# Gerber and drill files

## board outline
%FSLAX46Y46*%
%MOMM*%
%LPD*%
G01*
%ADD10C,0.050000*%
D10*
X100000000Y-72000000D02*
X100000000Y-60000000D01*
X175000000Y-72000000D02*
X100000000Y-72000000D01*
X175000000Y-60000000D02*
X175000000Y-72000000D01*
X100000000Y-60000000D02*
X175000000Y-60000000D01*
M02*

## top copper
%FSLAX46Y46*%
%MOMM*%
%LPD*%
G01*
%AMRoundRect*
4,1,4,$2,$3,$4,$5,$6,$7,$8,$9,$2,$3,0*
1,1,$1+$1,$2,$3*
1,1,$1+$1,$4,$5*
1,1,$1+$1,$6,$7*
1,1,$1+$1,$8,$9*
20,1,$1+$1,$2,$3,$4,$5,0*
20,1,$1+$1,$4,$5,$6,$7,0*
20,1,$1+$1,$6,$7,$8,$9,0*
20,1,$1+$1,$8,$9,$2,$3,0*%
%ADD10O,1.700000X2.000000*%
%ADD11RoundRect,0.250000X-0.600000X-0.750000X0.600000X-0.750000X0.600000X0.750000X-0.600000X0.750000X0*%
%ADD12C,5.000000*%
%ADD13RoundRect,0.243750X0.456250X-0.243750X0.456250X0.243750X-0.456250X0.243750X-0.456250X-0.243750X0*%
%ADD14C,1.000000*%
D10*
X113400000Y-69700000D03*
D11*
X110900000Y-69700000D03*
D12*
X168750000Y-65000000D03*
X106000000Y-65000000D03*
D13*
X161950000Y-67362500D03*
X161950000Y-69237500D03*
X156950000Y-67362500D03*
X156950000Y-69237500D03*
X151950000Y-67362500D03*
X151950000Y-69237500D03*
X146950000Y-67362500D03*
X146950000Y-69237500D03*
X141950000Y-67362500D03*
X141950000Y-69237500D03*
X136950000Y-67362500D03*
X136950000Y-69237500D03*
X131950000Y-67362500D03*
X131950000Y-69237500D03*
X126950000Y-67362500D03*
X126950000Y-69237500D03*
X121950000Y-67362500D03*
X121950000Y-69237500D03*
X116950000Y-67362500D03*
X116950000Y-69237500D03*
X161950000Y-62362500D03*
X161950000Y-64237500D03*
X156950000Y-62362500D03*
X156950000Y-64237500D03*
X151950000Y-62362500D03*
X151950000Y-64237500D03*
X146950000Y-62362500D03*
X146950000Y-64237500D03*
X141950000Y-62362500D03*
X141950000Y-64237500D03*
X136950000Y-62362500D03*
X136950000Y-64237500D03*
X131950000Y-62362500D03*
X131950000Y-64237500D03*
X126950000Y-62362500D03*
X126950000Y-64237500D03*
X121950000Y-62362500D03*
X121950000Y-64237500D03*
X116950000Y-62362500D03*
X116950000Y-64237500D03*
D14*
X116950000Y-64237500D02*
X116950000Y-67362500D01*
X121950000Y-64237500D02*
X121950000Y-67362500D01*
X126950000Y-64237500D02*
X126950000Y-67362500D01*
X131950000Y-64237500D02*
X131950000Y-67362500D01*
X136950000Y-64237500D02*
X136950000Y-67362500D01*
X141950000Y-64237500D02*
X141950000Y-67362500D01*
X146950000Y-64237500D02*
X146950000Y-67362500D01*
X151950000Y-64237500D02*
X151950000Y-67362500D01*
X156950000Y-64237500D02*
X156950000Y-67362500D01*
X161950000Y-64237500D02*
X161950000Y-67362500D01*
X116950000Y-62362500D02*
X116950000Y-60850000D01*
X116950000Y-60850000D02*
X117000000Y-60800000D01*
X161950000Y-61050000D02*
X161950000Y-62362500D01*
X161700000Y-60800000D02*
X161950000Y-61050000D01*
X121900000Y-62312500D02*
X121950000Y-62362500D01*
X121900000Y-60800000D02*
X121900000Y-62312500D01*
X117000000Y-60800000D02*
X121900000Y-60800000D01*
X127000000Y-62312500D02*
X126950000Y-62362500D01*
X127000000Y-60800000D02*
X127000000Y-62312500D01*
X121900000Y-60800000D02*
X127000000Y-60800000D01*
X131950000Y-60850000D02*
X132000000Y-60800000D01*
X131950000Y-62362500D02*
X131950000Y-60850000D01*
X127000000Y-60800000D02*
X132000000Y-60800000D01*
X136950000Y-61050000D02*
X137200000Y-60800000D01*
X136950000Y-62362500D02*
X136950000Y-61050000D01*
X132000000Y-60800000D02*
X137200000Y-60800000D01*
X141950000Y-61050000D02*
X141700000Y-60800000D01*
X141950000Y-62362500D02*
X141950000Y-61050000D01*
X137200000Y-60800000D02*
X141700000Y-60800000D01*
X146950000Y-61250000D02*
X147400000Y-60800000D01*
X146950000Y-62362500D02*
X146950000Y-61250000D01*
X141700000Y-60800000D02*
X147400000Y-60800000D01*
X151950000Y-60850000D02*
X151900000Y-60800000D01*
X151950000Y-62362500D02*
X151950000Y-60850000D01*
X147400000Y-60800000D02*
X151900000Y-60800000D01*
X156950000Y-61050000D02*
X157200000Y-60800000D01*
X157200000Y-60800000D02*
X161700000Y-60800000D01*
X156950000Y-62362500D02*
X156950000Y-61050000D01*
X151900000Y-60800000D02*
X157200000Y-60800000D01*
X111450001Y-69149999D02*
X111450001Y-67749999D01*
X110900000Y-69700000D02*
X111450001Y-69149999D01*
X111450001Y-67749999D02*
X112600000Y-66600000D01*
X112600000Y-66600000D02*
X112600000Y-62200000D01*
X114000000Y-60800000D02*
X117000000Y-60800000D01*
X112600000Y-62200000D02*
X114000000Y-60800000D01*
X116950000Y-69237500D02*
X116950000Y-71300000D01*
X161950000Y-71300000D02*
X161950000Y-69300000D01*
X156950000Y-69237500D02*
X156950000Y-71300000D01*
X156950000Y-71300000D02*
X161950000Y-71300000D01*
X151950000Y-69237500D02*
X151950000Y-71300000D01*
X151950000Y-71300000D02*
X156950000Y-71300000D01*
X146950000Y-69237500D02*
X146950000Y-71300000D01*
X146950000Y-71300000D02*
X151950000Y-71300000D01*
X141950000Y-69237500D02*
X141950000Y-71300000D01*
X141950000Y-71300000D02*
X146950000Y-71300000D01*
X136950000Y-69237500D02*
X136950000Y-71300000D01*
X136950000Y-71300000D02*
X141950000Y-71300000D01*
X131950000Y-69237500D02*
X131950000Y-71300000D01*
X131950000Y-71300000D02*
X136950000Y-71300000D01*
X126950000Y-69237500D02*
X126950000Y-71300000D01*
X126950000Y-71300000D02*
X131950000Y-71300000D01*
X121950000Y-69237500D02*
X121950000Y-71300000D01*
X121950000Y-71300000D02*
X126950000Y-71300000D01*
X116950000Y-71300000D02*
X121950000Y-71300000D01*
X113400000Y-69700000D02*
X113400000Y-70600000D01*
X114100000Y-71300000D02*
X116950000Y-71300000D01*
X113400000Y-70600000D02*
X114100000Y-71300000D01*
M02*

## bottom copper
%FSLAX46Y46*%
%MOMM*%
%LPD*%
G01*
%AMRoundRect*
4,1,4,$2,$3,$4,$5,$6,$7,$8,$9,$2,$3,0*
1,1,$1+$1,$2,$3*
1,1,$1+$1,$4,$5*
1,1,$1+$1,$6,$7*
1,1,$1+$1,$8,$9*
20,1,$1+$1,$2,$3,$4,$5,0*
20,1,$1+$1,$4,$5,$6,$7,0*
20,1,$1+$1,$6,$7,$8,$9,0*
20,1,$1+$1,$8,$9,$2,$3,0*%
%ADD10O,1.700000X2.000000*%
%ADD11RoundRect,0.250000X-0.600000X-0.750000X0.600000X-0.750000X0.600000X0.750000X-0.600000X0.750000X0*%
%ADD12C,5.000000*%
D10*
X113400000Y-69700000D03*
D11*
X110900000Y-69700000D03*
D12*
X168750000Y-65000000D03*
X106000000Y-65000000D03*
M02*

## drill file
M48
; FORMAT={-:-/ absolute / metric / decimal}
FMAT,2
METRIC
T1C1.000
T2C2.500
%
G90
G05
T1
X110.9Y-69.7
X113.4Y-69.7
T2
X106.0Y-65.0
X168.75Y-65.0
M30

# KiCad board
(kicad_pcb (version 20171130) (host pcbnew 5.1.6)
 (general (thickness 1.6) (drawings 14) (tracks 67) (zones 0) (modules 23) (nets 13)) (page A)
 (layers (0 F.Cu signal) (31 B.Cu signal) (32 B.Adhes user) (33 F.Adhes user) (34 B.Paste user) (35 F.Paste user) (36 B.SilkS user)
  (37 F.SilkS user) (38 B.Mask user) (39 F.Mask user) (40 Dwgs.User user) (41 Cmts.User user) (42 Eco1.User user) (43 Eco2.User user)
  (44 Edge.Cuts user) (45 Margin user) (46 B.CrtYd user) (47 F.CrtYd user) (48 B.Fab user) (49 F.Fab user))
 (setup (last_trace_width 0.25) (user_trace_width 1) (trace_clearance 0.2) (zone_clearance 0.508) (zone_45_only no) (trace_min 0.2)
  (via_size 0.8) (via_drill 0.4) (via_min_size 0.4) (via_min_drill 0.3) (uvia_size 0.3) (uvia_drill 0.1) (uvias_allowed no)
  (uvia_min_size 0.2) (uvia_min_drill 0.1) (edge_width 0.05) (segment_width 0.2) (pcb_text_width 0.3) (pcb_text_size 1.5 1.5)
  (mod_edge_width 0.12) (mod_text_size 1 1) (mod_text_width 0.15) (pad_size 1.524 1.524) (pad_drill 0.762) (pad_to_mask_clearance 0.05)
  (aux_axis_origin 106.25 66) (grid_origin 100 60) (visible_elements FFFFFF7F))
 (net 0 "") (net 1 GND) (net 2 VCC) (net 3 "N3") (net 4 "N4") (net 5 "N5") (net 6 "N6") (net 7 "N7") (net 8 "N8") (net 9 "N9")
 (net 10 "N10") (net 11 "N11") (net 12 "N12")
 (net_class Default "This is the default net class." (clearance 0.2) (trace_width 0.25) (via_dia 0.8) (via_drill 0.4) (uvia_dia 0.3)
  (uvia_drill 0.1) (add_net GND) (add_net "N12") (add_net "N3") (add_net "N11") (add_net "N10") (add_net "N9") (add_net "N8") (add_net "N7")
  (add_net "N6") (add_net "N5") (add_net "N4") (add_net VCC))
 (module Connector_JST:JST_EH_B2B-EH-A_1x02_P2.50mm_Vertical (layer F.Cu) (at 110.9 69.7)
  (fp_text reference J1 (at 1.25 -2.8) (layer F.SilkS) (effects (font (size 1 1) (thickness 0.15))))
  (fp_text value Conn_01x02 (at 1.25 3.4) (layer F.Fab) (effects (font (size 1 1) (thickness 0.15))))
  (pad 2 thru_hole oval (at 2.5 0) (size 1.7 2) (drill 1) (layers *.Cu *.Mask) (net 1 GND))
  (pad 1 thru_hole roundrect (at 0 0) (size 1.7 2) (drill 1) (layers *.Cu *.Mask) (roundrect_rratio 0.147059) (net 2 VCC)))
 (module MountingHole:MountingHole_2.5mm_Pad (layer F.Cu) (at 168.75 65)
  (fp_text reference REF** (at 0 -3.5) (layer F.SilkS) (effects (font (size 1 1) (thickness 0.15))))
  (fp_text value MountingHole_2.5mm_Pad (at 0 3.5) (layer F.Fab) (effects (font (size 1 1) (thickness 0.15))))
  (pad 1 thru_hole circle (at 0 0) (size 5 5) (drill 2.5) (layers *.Cu *.Mask)))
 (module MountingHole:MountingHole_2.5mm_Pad (layer F.Cu) (at 106 65)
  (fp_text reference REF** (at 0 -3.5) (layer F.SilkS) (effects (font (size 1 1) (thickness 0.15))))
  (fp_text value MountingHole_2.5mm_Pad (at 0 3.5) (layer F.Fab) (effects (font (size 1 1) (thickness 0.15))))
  (pad 1 thru_hole circle (at 0 0) (size 5 5) (drill 2.5) (layers *.Cu *.Mask)))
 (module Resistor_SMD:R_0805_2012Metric (layer F.Cu) (at 161.95 68.3 90)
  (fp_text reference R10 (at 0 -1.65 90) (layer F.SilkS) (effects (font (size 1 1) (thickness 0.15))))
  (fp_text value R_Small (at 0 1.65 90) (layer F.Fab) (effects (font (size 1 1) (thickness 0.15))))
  (pad 2 smd roundrect (at 0.9375 0 90) (size 0.975 1.4) (layers F.Cu F.Paste F.Mask) (roundrect_rratio 0.25) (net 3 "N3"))
  (pad 1 smd roundrect (at -0.9375 0 90) (size 0.975 1.4) (layers F.Cu F.Paste F.Mask) (roundrect_rratio 0.25) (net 1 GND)))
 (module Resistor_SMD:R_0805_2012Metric (layer F.Cu) (at 156.95 68.3 90)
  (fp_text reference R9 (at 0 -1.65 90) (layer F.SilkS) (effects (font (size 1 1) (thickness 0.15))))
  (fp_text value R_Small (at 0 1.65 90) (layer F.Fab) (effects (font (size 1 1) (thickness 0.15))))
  (pad 2 smd roundrect (at 0.9375 0 90) (size 0.975 1.4) (layers F.Cu F.Paste F.Mask) (roundrect_rratio 0.25) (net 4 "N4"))
  (pad 1 smd roundrect (at -0.9375 0 90) (size 0.975 1.4) (layers F.Cu F.Paste F.Mask) (roundrect_rratio 0.25) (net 1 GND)))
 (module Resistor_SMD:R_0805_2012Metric (layer F.Cu) (at 151.95 68.3 90)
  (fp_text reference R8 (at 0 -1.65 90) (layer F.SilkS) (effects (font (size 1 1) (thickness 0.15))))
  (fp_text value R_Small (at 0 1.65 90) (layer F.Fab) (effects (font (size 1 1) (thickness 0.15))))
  (pad 2 smd roundrect (at 0.9375 0 90) (size 0.975 1.4) (layers F.Cu F.Paste F.Mask) (roundrect_rratio 0.25) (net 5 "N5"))
  (pad 1 smd roundrect (at -0.9375 0 90) (size 0.975 1.4) (layers F.Cu F.Paste F.Mask) (roundrect_rratio 0.25) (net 1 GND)))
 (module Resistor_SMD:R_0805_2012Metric (layer F.Cu) (at 146.95 68.3 90)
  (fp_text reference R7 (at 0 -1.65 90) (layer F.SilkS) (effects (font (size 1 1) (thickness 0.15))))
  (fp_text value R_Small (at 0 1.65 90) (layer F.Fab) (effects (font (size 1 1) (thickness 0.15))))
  (pad 2 smd roundrect (at 0.9375 0 90) (size 0.975 1.4) (layers F.Cu F.Paste F.Mask) (roundrect_rratio 0.25) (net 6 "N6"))
  (pad 1 smd roundrect (at -0.9375 0 90) (size 0.975 1.4) (layers F.Cu F.Paste F.Mask) (roundrect_rratio 0.25) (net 1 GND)))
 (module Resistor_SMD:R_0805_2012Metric (layer F.Cu) (at 141.95 68.3 90)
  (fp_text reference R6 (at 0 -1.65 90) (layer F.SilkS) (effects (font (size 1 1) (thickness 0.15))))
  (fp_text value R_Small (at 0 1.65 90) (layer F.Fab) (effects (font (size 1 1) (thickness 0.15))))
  (pad 2 smd roundrect (at 0.9375 0 90) (size 0.975 1.4) (layers F.Cu F.Paste F.Mask) (roundrect_rratio 0.25) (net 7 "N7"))
  (pad 1 smd roundrect (at -0.9375 0 90) (size 0.975 1.4) (layers F.Cu F.Paste F.Mask) (roundrect_rratio 0.25) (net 1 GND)))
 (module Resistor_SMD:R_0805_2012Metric (layer F.Cu) (at 136.95 68.3 90)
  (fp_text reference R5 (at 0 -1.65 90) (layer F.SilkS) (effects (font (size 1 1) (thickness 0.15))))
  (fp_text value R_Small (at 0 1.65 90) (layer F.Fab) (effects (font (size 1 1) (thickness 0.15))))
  (pad 2 smd roundrect (at 0.9375 0 90) (size 0.975 1.4) (layers F.Cu F.Paste F.Mask) (roundrect_rratio 0.25) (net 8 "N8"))
  (pad 1 smd roundrect (at -0.9375 0 90) (size 0.975 1.4) (layers F.Cu F.Paste F.Mask) (roundrect_rratio 0.25) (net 1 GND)))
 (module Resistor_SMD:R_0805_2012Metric (layer F.Cu) (at 131.95 68.3 90)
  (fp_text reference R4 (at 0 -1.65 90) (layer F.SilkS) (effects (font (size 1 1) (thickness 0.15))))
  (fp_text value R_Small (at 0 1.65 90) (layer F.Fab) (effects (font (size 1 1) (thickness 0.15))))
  (pad 2 smd roundrect (at 0.9375 0 90) (size 0.975 1.4) (layers F.Cu F.Paste F.Mask) (roundrect_rratio 0.25) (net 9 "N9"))
  (pad 1 smd roundrect (at -0.9375 0 90) (size 0.975 1.4) (layers F.Cu F.Paste F.Mask) (roundrect_rratio 0.25) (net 1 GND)))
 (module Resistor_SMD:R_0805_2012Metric (layer F.Cu) (at 126.95 68.3 90)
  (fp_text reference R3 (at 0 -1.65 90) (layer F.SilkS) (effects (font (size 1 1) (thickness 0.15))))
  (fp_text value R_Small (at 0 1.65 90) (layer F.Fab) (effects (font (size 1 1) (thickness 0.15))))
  (pad 2 smd roundrect (at 0.9375 0 90) (size 0.975 1.4) (layers F.Cu F.Paste F.Mask) (roundrect_rratio 0.25) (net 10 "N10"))
  (pad 1 smd roundrect (at -0.9375 0 90) (size 0.975 1.4) (layers F.Cu F.Paste F.Mask) (roundrect_rratio 0.25) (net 1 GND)))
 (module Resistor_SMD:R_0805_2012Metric (layer F.Cu) (at 121.95 68.3 90)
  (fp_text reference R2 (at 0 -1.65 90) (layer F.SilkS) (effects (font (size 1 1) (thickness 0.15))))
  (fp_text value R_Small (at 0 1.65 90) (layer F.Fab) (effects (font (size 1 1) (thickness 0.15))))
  (pad 2 smd roundrect (at 0.9375 0 90) (size 0.975 1.4) (layers F.Cu F.Paste F.Mask) (roundrect_rratio 0.25) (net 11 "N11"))
  (pad 1 smd roundrect (at -0.9375 0 90) (size 0.975 1.4) (layers F.Cu F.Paste F.Mask) (roundrect_rratio 0.25) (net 1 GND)))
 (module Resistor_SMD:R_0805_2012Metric (layer F.Cu) (at 116.95 68.3 90)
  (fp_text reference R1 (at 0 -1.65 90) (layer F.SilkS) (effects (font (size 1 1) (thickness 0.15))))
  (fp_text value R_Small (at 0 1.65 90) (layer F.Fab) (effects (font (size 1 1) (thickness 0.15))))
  (pad 2 smd roundrect (at 0.9375 0 90) (size 0.975 1.4) (layers F.Cu F.Paste F.Mask) (roundrect_rratio 0.25) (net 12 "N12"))
  (pad 1 smd roundrect (at -0.9375 0 90) (size 0.975 1.4) (layers F.Cu F.Paste F.Mask) (roundrect_rratio 0.25) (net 1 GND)))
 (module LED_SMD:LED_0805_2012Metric (layer F.Cu) (at 161.95 63.3 90)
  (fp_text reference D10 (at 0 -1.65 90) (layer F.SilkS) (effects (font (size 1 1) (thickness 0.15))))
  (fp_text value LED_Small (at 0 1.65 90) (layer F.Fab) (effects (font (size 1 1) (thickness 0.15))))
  (pad 2 smd roundrect (at 0.9375 0 90) (size 0.975 1.4) (layers F.Cu F.Paste F.Mask) (roundrect_rratio 0.25) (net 2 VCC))
  (pad 1 smd roundrect (at -0.9375 0 90) (size 0.975 1.4) (layers F.Cu F.Paste F.Mask) (roundrect_rratio 0.25) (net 3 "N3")))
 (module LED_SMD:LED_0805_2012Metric (layer F.Cu) (at 156.95 63.3 90)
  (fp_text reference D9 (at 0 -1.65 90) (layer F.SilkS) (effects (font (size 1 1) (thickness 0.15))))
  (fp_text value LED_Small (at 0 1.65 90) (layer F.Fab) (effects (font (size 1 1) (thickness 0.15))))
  (pad 2 smd roundrect (at 0.9375 0 90) (size 0.975 1.4) (layers F.Cu F.Paste F.Mask) (roundrect_rratio 0.25) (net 2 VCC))
  (pad 1 smd roundrect (at -0.9375 0 90) (size 0.975 1.4) (layers F.Cu F.Paste F.Mask) (roundrect_rratio 0.25) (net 4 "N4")))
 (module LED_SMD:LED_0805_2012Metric (layer F.Cu) (at 151.95 63.3 90)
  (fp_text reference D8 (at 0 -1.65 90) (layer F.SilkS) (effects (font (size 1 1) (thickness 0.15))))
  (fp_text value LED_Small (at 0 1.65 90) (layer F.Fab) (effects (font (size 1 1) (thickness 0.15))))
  (pad 2 smd roundrect (at 0.9375 0 90) (size 0.975 1.4) (layers F.Cu F.Paste F.Mask) (roundrect_rratio 0.25) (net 2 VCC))
  (pad 1 smd roundrect (at -0.9375 0 90) (size 0.975 1.4) (layers F.Cu F.Paste F.Mask) (roundrect_rratio 0.25) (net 5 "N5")))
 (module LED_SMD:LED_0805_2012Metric (layer F.Cu) (at 146.95 63.3 90)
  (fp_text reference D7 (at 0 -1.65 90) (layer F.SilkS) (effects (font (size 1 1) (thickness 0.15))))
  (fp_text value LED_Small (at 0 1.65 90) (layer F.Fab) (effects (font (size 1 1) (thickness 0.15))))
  (pad 2 smd roundrect (at 0.9375 0 90) (size 0.975 1.4) (layers F.Cu F.Paste F.Mask) (roundrect_rratio 0.25) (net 2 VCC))
  (pad 1 smd roundrect (at -0.9375 0 90) (size 0.975 1.4) (layers F.Cu F.Paste F.Mask) (roundrect_rratio 0.25) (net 6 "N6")))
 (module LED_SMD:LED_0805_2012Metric (layer F.Cu) (at 141.95 63.3 90)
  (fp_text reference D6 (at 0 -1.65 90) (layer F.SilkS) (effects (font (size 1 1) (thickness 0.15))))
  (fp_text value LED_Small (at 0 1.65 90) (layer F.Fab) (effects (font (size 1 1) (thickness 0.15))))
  (pad 2 smd roundrect (at 0.9375 0 90) (size 0.975 1.4) (layers F.Cu F.Paste F.Mask) (roundrect_rratio 0.25) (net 2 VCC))
  (pad 1 smd roundrect (at -0.9375 0 90) (size 0.975 1.4) (layers F.Cu F.Paste F.Mask) (roundrect_rratio 0.25) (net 7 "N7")))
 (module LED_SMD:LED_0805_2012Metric (layer F.Cu) (at 136.95 63.3 90)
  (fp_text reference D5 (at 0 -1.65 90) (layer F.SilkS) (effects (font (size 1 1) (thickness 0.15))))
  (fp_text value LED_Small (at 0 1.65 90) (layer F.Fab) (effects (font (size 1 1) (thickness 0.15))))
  (pad 2 smd roundrect (at 0.9375 0 90) (size 0.975 1.4) (layers F.Cu F.Paste F.Mask) (roundrect_rratio 0.25) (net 2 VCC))
  (pad 1 smd roundrect (at -0.9375 0 90) (size 0.975 1.4) (layers F.Cu F.Paste F.Mask) (roundrect_rratio 0.25) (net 8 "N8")))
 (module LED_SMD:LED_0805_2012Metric (layer F.Cu) (at 131.95 63.3 90)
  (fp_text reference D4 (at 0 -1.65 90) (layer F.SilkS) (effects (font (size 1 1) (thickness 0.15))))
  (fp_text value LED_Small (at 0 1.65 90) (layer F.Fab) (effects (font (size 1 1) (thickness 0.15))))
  (pad 2 smd roundrect (at 0.9375 0 90) (size 0.975 1.4) (layers F.Cu F.Paste F.Mask) (roundrect_rratio 0.25) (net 2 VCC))
  (pad 1 smd roundrect (at -0.9375 0 90) (size 0.975 1.4) (layers F.Cu F.Paste F.Mask) (roundrect_rratio 0.25) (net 9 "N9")))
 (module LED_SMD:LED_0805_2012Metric (layer F.Cu) (at 126.95 63.3 90)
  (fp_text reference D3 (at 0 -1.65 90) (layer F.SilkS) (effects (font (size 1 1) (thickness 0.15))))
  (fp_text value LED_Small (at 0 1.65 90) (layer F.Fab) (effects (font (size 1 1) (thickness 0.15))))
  (pad 2 smd roundrect (at 0.9375 0 90) (size 0.975 1.4) (layers F.Cu F.Paste F.Mask) (roundrect_rratio 0.25) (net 2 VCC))
  (pad 1 smd roundrect (at -0.9375 0 90) (size 0.975 1.4) (layers F.Cu F.Paste F.Mask) (roundrect_rratio 0.25) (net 10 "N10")))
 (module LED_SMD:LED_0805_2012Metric (layer F.Cu) (at 121.95 63.3 90)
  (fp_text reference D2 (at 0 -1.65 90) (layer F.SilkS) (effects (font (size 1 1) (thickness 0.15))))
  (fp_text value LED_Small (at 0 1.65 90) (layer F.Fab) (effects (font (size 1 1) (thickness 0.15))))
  (pad 2 smd roundrect (at 0.9375 0 90) (size 0.975 1.4) (layers F.Cu F.Paste F.Mask) (roundrect_rratio 0.25) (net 2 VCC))
  (pad 1 smd roundrect (at -0.9375 0 90) (size 0.975 1.4) (layers F.Cu F.Paste F.Mask) (roundrect_rratio 0.25) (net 11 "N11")))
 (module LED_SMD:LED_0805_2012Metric (layer F.Cu) (at 116.95 63.3 90)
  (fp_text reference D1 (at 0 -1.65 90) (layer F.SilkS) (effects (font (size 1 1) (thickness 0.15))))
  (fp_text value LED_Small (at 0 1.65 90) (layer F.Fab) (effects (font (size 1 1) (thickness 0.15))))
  (pad 2 smd roundrect (at 0.9375 0 90) (size 0.975 1.4) (layers F.Cu F.Paste F.Mask) (roundrect_rratio 0.25) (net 2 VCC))
  (pad 1 smd roundrect (at -0.9375 0 90) (size 0.975 1.4) (layers F.Cu F.Paste F.Mask) (roundrect_rratio 0.25) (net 12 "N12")))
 (gr_line (start 100 72) (end 100 60) (layer Edge.Cuts) (width 0.05))
 (gr_line (start 175 72) (end 100 72) (layer Edge.Cuts) (width 0.05))
 (gr_line (start 175 60) (end 175 72) (layer Edge.Cuts) (width 0.05))
 (gr_line (start 100 60) (end 175 60) (layer Edge.Cuts) (width 0.05))
 (segment (start 116.95 64.2375) (end 116.95 67.3625) (width 1) (layer F.Cu) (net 12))
 (segment (start 121.95 64.2375) (end 121.95 67.3625) (width 1) (layer F.Cu) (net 11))
 (segment (start 126.95 64.2375) (end 126.95 67.3625) (width 1) (layer F.Cu) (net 10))
 (segment (start 131.95 64.2375) (end 131.95 67.3625) (width 1) (layer F.Cu) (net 9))
 (segment (start 136.95 64.2375) (end 136.95 67.3625) (width 1) (layer F.Cu) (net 8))
 (segment (start 141.95 64.2375) (end 141.95 67.3625) (width 1) (layer F.Cu) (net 7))
 (segment (start 146.95 64.2375) (end 146.95 67.3625) (width 1) (layer F.Cu) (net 6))
 (segment (start 151.95 64.2375) (end 151.95 67.3625) (width 1) (layer F.Cu) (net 5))
 (segment (start 156.95 64.2375) (end 156.95 67.3625) (width 1) (layer F.Cu) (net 4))
 (segment (start 161.95 64.2375) (end 161.95 67.3625) (width 1) (layer F.Cu) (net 3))
 (segment (start 116.95 62.3625) (end 116.95 60.85) (width 1) (layer F.Cu) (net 2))
 (segment (start 116.95 60.85) (end 117 60.8) (width 1) (layer F.Cu) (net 2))
 (segment (start 161.95 61.05) (end 161.95 62.3625) (width 1) (layer F.Cu) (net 2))
 (segment (start 161.7 60.8) (end 161.95 61.05) (width 1) (layer F.Cu) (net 2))
 (segment (start 121.9 62.3125) (end 121.95 62.3625) (width 1) (layer F.Cu) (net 2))
 (segment (start 121.9 60.8) (end 121.9 62.3125) (width 1) (layer F.Cu) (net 2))
 (segment (start 117 60.8) (end 121.9 60.8) (width 1) (layer F.Cu) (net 2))
 (segment (start 127 62.3125) (end 126.95 62.3625) (width 1) (layer F.Cu) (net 2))
 (segment (start 127 60.8) (end 127 62.3125) (width 1) (layer F.Cu) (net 2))
 (segment (start 121.9 60.8) (end 127 60.8) (width 1) (layer F.Cu) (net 2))
 (segment (start 131.95 60.85) (end 132 60.8) (width 1) (layer F.Cu) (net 2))
 (segment (start 131.95 62.3625) (end 131.95 60.85) (width 1) (layer F.Cu) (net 2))
 (segment (start 127 60.8) (end 132 60.8) (width 1) (layer F.Cu) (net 2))
 (segment (start 136.95 61.05) (end 137.2 60.8) (width 1) (layer F.Cu) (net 2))
 (segment (start 136.95 62.3625) (end 136.95 61.05) (width 1) (layer F.Cu) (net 2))
 (segment (start 132 60.8) (end 137.2 60.8) (width 1) (layer F.Cu) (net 2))
 (segment (start 141.95 61.05) (end 141.7 60.8) (width 1) (layer F.Cu) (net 2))
 (segment (start 141.95 62.3625) (end 141.95 61.05) (width 1) (layer F.Cu) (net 2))
 (segment (start 137.2 60.8) (end 141.7 60.8) (width 1) (layer F.Cu) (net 2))
 (segment (start 146.95 61.25) (end 147.4 60.8) (width 1) (layer F.Cu) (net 2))
 (segment (start 146.95 62.3625) (end 146.95 61.25) (width 1) (layer F.Cu) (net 2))
 (segment (start 141.7 60.8) (end 147.4 60.8) (width 1) (layer F.Cu) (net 2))
 (segment (start 151.95 60.85) (end 151.9 60.8) (width 1) (layer F.Cu) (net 2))
 (segment (start 151.95 62.3625) (end 151.95 60.85) (width 1) (layer F.Cu) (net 2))
 (segment (start 147.4 60.8) (end 151.9 60.8) (width 1) (layer F.Cu) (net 2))
 (segment (start 156.95 61.05) (end 157.2 60.8) (width 1) (layer F.Cu) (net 2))
 (segment (start 157.2 60.8) (end 161.7 60.8) (width 1) (layer F.Cu) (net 2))
 (segment (start 156.95 62.3625) (end 156.95 61.05) (width 1) (layer F.Cu) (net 2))
 (segment (start 151.9 60.8) (end 157.2 60.8) (width 1) (layer F.Cu) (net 2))
 (segment (start 111.450001 69.149999) (end 111.450001 67.749999) (width 1) (layer F.Cu) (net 2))
 (segment (start 110.9 69.7) (end 111.450001 69.149999) (width 1) (layer F.Cu) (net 2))
 (segment (start 111.450001 67.749999) (end 112.6 66.6) (width 1) (layer F.Cu) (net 2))
 (segment (start 112.6 66.6) (end 112.6 62.2) (width 1) (layer F.Cu) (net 2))
 (segment (start 114 60.8) (end 117 60.8) (width 1) (layer F.Cu) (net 2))
 (segment (start 112.6 62.2) (end 114 60.8) (width 1) (layer F.Cu) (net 2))
 (segment (start 116.95 69.2375) (end 116.95 71.3) (width 1) (layer F.Cu) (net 1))
 (segment (start 161.95 71.3) (end 161.95 69.3) (width 1) (layer F.Cu) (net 1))
 (segment (start 156.95 69.2375) (end 156.95 71.3) (width 1) (layer F.Cu) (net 1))
 (segment (start 156.95 71.3) (end 161.95 71.3) (width 1) (layer F.Cu) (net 1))
 (segment (start 151.95 69.2375) (end 151.95 71.3) (width 1) (layer F.Cu) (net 1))
 (segment (start 151.95 71.3) (end 156.95 71.3) (width 1) (layer F.Cu) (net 1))
 (segment (start 146.95 69.2375) (end 146.95 71.3) (width 1) (layer F.Cu) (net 1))
 (segment (start 146.95 71.3) (end 151.95 71.3) (width 1) (layer F.Cu) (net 1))
 (segment (start 141.95 69.2375) (end 141.95 71.3) (width 1) (layer F.Cu) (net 1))
 (segment (start 141.95 71.3) (end 146.95 71.3) (width 1) (layer F.Cu) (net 1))
 (segment (start 136.95 69.2375) (end 136.95 71.3) (width 1) (layer F.Cu) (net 1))
 (segment (start 136.95 71.3) (end 141.95 71.3) (width 1) (layer F.Cu) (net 1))
 (segment (start 131.95 69.2375) (end 131.95 71.3) (width 1) (layer F.Cu) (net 1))
 (segment (start 131.95 71.3) (end 136.95 71.3) (width 1) (layer F.Cu) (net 1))
 (segment (start 126.95 69.2375) (end 126.95 71.3) (width 1) (layer F.Cu) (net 1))
 (segment (start 126.95 71.3) (end 131.95 71.3) (width 1) (layer F.Cu) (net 1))
 (segment (start 121.95 69.2375) (end 121.95 71.3) (width 1) (layer F.Cu) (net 1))
 (segment (start 121.95 71.3) (end 126.95 71.3) (width 1) (layer F.Cu) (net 1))
 (segment (start 116.95 71.3) (end 121.95 71.3) (width 1) (layer F.Cu) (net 1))
 (segment (start 113.4 69.7) (end 113.4 70.6) (width 1) (layer F.Cu) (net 1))
 (segment (start 114.1 71.3) (end 116.95 71.3) (width 1) (layer F.Cu) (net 1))
 (segment (start 113.4 70.6) (end 114.1 71.3) (width 1) (layer F.Cu) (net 1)))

